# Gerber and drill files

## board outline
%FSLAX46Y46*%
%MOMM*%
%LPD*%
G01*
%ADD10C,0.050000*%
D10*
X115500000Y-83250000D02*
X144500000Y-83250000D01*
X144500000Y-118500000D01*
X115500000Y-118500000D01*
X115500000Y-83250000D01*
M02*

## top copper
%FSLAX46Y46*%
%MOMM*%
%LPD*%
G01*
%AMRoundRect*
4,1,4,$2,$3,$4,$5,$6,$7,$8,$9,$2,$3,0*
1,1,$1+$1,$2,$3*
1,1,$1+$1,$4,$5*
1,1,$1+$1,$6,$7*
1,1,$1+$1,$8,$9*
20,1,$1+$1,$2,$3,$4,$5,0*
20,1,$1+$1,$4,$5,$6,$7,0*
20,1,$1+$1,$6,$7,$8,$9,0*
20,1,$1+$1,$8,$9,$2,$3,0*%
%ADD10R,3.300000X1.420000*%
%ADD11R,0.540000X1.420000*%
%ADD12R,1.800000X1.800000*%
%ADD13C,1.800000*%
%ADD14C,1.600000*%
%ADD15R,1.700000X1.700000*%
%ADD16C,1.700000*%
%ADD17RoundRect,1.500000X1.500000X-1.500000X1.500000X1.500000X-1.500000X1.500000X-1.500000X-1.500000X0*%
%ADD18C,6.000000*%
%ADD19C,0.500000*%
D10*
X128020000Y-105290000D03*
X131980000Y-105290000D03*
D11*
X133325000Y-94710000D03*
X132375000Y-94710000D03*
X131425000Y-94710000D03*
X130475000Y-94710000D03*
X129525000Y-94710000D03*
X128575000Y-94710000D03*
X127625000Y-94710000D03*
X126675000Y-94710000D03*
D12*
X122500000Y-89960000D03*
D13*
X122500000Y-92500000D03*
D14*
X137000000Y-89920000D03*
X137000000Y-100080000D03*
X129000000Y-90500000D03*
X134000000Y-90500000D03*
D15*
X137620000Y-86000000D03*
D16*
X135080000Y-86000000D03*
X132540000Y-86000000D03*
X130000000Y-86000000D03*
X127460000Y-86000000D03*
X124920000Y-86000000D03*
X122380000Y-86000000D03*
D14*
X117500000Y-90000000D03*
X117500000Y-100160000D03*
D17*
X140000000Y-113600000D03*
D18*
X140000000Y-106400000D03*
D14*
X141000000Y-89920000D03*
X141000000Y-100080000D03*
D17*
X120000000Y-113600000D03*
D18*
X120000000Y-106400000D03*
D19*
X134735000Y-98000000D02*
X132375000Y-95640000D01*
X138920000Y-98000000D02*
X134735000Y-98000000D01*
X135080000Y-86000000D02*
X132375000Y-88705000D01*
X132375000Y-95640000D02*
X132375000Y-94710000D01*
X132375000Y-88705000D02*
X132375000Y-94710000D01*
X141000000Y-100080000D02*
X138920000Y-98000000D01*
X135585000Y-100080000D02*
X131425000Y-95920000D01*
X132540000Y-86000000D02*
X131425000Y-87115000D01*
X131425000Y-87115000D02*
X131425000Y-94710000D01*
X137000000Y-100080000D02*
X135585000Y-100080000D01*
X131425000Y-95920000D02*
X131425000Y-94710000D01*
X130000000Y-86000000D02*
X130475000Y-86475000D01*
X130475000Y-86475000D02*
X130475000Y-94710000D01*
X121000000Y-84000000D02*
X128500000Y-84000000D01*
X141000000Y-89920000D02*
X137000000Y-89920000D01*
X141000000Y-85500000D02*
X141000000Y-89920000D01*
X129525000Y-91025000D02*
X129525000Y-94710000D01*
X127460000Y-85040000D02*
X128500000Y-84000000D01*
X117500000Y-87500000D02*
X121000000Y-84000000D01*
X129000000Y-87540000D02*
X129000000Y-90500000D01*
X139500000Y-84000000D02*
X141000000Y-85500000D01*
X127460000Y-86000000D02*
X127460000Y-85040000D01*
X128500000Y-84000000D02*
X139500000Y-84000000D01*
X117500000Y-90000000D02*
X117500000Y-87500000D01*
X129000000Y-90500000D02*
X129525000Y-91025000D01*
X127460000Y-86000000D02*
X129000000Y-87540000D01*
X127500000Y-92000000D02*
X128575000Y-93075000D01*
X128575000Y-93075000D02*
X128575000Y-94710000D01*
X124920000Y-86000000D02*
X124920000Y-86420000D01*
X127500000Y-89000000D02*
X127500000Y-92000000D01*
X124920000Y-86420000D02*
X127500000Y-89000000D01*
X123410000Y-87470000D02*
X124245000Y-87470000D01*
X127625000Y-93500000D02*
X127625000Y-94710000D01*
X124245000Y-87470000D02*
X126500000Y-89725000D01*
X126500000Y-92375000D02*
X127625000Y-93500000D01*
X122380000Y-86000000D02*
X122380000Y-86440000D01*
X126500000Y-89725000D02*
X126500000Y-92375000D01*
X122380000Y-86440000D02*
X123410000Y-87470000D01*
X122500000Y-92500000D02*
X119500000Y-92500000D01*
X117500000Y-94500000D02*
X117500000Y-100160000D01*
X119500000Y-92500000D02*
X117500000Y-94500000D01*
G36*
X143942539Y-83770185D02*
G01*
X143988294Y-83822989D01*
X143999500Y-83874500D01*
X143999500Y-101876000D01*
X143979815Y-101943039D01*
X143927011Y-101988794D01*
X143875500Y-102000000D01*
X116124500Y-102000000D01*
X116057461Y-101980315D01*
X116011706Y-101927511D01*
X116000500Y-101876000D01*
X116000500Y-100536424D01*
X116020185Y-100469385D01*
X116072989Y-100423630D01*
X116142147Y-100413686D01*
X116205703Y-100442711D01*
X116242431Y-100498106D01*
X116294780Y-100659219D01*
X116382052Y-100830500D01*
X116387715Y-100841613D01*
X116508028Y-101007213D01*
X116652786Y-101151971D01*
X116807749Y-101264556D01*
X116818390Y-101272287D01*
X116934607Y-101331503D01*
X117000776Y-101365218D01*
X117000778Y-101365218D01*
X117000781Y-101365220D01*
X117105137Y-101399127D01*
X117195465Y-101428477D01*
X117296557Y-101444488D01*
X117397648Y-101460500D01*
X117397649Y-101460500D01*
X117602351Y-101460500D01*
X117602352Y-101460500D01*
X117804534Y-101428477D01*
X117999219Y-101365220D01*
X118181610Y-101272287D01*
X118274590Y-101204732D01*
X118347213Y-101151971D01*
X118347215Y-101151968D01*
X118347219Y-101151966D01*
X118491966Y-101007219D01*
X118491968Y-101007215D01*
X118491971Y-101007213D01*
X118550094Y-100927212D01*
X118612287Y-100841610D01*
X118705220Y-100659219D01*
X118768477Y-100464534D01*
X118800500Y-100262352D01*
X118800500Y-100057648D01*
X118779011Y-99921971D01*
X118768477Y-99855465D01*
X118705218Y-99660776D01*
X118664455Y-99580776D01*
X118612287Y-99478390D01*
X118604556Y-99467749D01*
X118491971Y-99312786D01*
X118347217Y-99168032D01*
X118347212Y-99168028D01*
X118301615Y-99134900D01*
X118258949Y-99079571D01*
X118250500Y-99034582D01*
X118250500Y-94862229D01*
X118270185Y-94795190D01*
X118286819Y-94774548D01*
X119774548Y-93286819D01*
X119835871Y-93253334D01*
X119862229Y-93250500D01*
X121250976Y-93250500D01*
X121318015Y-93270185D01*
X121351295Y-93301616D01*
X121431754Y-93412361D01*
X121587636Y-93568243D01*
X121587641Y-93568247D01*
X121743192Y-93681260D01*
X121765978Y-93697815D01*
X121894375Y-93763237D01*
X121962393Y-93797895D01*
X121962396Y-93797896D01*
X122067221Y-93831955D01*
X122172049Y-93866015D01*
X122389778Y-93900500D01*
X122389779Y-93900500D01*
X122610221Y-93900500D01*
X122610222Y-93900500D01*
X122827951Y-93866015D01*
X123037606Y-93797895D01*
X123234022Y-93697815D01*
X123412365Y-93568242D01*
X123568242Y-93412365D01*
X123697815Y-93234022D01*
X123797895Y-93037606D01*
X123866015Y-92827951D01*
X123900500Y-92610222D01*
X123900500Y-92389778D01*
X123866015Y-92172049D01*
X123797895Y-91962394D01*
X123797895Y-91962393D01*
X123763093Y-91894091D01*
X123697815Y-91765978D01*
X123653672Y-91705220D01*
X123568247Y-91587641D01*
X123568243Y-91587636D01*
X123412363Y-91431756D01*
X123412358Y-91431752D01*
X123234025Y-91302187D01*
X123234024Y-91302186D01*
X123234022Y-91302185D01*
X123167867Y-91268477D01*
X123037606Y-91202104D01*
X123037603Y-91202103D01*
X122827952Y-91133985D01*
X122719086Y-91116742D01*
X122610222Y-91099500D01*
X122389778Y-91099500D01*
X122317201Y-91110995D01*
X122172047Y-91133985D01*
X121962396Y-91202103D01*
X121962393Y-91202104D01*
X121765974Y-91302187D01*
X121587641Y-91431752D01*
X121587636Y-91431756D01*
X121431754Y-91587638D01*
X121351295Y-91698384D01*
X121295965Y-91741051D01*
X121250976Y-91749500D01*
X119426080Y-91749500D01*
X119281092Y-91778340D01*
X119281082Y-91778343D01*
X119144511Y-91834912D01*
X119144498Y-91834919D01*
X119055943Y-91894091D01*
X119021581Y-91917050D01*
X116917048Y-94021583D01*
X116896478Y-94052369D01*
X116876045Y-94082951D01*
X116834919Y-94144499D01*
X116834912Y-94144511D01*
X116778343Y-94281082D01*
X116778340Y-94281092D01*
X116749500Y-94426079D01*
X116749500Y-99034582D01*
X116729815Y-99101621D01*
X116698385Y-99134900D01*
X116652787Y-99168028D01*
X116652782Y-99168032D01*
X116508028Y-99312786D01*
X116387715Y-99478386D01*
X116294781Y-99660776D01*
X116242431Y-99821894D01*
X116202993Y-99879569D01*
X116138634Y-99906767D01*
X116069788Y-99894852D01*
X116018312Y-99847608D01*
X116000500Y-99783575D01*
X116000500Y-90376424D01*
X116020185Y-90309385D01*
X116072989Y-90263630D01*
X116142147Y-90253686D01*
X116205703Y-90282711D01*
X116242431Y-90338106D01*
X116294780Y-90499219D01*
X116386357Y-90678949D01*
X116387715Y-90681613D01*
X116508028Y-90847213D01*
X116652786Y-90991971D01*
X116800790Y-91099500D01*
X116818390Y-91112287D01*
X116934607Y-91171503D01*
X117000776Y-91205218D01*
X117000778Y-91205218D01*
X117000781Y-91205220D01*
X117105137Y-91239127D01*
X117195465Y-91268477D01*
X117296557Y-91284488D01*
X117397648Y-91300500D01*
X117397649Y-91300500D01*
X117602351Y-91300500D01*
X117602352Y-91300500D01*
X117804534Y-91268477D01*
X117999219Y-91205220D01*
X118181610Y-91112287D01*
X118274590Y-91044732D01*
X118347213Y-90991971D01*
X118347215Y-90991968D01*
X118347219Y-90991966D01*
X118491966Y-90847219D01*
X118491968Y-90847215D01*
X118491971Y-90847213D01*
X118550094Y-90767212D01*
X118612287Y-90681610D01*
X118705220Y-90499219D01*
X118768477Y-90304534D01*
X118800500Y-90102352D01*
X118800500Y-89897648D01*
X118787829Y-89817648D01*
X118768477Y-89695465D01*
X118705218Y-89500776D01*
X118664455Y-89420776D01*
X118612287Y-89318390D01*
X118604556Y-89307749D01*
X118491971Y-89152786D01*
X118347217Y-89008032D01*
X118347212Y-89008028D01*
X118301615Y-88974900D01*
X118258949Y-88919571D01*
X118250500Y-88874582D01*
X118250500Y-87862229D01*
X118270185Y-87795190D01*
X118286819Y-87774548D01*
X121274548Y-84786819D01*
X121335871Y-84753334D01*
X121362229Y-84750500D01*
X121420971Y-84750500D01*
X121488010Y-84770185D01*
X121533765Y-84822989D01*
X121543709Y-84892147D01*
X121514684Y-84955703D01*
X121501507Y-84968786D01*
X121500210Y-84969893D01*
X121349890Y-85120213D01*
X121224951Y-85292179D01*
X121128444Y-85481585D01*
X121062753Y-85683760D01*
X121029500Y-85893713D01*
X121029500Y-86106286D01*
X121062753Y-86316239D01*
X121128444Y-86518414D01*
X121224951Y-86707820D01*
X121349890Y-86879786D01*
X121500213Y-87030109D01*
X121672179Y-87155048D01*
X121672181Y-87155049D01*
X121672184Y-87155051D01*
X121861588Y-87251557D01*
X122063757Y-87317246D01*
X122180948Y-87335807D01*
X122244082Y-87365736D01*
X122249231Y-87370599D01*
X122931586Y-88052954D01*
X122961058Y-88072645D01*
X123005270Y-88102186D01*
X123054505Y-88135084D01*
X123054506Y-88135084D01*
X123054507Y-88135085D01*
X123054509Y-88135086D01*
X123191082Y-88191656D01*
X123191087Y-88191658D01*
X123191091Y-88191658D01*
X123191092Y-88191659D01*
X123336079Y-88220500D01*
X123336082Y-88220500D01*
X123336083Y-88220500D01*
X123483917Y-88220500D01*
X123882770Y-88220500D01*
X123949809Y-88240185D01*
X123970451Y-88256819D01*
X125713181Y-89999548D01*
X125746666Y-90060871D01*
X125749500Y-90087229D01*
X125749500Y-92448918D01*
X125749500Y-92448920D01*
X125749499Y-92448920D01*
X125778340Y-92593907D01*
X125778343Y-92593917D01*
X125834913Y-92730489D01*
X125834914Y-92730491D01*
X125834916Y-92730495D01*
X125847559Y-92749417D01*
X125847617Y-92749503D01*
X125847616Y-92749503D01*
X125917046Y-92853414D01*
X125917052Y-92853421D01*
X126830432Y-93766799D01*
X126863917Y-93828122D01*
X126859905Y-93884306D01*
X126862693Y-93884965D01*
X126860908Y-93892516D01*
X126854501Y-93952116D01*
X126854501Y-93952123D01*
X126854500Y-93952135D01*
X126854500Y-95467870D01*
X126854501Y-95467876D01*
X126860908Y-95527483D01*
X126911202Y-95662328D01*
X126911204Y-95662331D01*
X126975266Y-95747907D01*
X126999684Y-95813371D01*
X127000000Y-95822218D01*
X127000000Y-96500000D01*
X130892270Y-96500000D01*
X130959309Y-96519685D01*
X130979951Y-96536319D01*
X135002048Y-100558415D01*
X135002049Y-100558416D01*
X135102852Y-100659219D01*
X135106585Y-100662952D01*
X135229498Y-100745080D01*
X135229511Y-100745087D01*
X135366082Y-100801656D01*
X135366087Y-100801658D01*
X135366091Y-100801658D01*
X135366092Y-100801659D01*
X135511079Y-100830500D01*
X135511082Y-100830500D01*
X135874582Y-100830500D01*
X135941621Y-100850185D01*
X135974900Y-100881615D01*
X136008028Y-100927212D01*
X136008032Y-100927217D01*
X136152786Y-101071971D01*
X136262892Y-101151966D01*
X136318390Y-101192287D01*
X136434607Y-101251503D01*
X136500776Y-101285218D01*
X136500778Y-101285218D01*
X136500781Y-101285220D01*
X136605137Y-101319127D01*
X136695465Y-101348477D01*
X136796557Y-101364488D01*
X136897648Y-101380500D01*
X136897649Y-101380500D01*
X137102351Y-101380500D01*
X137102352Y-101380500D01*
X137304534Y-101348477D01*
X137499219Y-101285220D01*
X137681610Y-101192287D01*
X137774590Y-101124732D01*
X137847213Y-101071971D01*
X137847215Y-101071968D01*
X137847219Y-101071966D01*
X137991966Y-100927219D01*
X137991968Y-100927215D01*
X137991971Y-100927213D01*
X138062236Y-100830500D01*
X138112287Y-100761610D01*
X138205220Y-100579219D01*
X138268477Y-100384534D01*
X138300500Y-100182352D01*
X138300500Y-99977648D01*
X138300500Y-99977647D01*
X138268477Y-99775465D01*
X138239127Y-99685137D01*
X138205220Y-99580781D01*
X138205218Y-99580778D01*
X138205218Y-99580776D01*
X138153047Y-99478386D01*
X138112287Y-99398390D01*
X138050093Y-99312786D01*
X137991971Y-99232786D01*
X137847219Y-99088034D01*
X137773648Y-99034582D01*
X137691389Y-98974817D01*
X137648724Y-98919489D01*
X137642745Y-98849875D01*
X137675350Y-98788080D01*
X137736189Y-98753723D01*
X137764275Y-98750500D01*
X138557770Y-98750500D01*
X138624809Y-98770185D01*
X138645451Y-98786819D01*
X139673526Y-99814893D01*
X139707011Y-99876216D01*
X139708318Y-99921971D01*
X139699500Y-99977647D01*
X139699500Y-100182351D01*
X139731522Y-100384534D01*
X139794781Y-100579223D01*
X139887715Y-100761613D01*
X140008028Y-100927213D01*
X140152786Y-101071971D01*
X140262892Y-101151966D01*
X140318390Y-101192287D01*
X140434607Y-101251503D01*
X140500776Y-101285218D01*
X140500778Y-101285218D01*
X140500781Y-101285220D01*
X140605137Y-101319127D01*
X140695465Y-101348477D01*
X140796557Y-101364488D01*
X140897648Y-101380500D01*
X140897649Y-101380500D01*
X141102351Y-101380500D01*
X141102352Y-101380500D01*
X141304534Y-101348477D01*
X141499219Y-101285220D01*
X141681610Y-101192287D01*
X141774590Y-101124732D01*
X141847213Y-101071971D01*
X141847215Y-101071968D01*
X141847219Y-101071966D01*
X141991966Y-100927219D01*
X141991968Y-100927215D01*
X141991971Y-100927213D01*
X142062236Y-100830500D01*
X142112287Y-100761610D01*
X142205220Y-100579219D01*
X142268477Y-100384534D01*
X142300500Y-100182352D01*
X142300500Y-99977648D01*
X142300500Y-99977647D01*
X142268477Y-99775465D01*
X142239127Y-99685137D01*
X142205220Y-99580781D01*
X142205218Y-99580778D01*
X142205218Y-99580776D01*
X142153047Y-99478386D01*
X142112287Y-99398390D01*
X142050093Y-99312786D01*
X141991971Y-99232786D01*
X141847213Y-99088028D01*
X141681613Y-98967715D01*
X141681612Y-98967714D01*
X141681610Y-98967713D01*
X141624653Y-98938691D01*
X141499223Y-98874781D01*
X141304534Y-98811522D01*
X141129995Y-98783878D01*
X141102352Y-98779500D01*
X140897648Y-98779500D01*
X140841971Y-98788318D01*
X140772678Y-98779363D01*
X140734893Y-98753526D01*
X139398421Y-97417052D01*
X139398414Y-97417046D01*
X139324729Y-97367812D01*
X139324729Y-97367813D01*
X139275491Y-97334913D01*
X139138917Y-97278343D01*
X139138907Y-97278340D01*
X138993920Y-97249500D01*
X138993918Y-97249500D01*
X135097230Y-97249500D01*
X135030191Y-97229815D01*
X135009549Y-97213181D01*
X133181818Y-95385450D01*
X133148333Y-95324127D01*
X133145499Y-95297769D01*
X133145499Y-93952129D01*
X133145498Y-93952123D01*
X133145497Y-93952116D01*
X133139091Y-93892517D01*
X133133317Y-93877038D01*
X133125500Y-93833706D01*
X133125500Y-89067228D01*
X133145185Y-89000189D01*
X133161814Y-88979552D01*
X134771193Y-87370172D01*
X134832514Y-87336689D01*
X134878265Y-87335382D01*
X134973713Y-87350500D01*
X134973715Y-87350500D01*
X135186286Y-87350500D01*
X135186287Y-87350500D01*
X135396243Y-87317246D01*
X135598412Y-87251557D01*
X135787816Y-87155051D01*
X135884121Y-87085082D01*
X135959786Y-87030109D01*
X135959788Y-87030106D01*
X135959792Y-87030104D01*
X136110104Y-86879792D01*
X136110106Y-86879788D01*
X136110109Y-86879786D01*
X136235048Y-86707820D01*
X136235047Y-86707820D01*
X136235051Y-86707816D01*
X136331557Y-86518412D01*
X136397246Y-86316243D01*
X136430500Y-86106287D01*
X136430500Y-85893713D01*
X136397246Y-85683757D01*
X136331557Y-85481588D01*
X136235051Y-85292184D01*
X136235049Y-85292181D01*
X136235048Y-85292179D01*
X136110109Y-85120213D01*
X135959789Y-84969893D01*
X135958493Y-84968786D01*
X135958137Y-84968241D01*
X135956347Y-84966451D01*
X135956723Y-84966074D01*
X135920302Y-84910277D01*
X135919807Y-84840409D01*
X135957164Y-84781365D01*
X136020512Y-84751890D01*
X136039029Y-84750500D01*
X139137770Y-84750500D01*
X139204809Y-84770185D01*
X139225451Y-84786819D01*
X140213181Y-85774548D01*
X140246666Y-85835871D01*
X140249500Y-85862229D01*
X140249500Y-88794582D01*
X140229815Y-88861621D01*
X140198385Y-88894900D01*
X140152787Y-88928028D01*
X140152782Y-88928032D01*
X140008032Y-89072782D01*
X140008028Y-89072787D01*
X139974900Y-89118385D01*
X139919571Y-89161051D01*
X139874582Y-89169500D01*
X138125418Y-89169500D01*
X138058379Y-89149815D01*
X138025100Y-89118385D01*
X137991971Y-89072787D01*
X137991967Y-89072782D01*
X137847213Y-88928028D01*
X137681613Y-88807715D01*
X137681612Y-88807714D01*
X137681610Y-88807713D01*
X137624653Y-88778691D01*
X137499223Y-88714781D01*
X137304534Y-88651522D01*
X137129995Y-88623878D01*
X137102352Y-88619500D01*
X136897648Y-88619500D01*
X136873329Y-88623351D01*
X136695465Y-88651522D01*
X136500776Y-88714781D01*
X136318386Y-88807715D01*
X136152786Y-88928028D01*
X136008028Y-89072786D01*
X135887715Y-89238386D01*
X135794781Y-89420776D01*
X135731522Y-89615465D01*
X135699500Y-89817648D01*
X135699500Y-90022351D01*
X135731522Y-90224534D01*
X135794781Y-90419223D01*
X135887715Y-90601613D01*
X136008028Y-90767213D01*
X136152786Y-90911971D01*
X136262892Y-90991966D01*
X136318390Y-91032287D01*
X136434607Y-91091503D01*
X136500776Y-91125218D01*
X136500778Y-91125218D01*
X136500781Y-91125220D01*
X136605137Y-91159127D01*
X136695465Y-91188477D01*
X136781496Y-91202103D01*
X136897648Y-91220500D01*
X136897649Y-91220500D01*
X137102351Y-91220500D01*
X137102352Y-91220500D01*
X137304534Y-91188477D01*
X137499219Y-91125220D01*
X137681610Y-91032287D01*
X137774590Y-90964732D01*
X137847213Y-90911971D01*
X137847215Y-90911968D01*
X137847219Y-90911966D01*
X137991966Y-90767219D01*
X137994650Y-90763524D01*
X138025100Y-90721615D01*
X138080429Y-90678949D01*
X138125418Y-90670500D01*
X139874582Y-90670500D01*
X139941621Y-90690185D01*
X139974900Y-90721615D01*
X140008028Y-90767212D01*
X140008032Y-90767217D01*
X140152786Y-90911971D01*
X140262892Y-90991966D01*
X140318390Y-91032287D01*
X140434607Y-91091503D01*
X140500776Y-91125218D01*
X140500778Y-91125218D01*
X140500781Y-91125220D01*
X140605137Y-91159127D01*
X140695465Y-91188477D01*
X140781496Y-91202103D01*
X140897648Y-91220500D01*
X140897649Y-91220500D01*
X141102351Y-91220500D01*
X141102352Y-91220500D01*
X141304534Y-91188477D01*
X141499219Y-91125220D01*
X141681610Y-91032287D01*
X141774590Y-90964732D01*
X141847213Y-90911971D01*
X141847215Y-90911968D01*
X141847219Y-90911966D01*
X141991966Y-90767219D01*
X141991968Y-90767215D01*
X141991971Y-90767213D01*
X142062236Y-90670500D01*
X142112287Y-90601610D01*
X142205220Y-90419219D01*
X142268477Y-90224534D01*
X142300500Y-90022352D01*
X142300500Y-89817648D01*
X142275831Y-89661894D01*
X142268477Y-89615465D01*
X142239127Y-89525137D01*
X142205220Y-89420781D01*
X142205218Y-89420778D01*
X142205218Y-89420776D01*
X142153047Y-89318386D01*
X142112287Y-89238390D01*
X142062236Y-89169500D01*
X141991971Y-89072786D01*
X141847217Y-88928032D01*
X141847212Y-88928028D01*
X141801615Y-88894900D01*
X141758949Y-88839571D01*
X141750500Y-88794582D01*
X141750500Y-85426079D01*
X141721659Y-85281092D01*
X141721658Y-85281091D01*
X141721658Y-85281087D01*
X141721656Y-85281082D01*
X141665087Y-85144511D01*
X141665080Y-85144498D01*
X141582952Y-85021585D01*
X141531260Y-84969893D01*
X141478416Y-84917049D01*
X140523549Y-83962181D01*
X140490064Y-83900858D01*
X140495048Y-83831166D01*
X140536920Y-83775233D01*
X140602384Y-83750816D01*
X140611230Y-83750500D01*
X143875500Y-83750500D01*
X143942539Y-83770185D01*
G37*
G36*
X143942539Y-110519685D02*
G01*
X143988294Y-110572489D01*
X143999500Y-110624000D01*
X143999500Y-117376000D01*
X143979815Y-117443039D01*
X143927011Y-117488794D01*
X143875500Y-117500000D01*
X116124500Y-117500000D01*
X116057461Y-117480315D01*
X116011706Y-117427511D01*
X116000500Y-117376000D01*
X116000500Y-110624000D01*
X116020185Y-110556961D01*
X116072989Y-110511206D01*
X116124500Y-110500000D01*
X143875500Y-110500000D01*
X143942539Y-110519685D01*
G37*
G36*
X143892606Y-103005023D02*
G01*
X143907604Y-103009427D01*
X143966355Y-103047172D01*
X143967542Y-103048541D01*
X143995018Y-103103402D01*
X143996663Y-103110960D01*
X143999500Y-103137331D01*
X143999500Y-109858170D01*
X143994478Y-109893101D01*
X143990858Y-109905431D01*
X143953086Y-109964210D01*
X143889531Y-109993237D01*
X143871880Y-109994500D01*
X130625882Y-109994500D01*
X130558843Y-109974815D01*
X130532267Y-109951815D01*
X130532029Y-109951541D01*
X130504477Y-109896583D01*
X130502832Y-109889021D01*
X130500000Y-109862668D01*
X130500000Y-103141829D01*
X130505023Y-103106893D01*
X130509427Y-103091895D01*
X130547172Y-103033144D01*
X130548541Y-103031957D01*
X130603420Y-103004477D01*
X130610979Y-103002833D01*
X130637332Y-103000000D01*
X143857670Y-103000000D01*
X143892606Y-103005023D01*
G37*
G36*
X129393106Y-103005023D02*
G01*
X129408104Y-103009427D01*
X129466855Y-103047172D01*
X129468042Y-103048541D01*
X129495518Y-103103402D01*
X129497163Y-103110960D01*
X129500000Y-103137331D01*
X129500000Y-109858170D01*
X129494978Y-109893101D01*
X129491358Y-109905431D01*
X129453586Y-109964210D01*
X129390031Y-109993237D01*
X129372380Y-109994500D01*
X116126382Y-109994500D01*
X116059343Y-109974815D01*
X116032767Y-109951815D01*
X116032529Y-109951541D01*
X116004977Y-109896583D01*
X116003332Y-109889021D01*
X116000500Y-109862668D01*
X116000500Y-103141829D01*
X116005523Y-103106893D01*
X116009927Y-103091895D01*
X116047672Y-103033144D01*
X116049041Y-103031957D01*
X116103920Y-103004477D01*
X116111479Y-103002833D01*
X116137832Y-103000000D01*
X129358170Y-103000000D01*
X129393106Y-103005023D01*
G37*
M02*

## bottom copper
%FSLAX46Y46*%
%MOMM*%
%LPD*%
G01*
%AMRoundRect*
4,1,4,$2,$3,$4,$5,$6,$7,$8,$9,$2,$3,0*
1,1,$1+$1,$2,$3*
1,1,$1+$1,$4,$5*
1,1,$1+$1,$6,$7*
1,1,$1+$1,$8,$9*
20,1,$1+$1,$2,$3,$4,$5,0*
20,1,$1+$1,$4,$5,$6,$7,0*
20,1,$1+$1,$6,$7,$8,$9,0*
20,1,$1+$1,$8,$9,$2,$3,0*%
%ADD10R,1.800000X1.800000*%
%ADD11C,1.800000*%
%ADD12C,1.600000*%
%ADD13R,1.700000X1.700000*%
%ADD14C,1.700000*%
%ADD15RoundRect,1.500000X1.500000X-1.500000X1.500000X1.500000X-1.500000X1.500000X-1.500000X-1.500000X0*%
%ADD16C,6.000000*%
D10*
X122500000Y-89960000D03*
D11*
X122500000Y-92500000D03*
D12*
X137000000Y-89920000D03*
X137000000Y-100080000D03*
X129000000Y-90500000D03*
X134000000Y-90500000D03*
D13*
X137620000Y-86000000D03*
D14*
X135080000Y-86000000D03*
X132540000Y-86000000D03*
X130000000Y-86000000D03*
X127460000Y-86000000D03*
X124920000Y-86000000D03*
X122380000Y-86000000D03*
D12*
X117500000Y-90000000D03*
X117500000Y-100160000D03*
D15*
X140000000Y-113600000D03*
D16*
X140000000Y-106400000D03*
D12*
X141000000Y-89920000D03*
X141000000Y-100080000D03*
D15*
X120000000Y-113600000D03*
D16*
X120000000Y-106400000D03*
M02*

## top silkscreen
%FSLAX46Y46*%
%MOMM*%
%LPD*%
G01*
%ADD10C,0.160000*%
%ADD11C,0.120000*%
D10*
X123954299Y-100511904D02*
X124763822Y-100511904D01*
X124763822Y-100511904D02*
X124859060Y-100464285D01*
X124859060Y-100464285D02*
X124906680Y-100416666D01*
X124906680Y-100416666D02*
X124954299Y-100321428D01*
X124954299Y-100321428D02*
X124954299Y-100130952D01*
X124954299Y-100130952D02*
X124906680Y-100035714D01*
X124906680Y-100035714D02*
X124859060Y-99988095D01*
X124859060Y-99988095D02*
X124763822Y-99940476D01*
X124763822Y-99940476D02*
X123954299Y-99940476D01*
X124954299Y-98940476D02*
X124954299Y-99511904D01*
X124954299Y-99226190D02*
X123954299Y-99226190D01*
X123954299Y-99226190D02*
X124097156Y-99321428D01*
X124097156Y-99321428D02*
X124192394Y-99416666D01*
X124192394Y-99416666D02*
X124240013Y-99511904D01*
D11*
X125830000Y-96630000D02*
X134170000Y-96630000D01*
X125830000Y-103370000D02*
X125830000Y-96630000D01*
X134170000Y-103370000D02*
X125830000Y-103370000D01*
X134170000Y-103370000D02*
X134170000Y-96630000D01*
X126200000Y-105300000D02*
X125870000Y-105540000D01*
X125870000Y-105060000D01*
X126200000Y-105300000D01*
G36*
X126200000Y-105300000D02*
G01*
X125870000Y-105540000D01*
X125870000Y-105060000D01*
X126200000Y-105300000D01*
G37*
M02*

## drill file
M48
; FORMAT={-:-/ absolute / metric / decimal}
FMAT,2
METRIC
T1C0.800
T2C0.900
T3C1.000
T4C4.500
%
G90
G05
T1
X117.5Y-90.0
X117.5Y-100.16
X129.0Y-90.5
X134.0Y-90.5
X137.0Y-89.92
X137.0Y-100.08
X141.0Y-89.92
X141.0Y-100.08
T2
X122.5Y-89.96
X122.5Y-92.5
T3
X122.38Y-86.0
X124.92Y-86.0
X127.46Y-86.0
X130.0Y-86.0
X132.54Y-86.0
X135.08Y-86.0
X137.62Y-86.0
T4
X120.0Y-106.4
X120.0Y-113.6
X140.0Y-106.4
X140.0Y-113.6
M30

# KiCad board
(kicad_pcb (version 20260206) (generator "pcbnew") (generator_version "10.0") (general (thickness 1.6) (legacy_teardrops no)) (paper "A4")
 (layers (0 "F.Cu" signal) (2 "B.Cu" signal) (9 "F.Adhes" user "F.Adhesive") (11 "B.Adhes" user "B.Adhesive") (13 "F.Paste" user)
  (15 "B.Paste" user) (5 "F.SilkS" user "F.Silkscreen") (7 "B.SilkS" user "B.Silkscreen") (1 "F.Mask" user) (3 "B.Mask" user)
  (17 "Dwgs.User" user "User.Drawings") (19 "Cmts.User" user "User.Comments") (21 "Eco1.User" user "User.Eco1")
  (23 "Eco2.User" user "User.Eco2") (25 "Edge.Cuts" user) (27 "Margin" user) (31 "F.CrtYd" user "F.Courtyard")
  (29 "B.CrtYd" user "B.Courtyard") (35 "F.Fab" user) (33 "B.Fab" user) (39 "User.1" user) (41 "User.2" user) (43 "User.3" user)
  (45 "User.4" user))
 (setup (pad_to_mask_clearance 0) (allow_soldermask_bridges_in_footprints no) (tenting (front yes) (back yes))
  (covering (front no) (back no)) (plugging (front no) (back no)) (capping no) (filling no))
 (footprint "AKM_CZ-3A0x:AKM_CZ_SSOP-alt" (layer "F.Cu") (at 130 100 90)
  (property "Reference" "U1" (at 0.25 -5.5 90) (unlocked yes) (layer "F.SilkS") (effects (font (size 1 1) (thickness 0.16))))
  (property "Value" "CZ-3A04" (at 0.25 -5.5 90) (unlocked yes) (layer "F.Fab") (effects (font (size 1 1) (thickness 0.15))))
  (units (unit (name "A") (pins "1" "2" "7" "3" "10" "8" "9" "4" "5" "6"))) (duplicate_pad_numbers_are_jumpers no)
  (fp_line (start 3.37 -4.17) (end 3.37 4.17) (stroke (width 0.12) (type solid)) (layer "F.SilkS"))
  (fp_line (start -3.37 -4.17) (end 3.37 -4.17) (stroke (width 0.12) (type solid)) (layer "F.SilkS"))
  (fp_line (start -3.37 4.17) (end -3.37 -4.17) (stroke (width 0.12) (type solid)) (layer "F.SilkS"))
  (fp_line (start -3.37 4.17) (end 3.37 4.17) (stroke (width 0.12) (type solid)) (layer "F.SilkS"))
  (fp_poly
   (pts (xy -5.3 -3.8) (xy -5.54 -4.13) (xy -5.06 -4.13) (xy -5.3 -3.8)) (stroke (width 0.12) (type solid)) (fill yes) (layer "F.SilkS"))
  (pad "1" smd rect (at -5.29 -1.98 270) (size 1.42 3.3) (layers "F.Cu" "F.Mask" "F.Paste") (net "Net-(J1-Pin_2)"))
  (pad "2" smd rect (at -5.29 1.98 270) (size 1.42 3.3) (layers "F.Cu" "F.Mask" "F.Paste") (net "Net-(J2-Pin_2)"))
  (pad "3" smd rect (at 5.29 3.325 270) (size 1.42 0.54) (layers "F.Cu" "F.Mask" "F.Paste") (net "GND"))
  (pad "4" smd rect (at 5.29 2.375 270) (size 1.42 0.54) (layers "F.Cu" "F.Mask" "F.Paste") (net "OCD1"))
  (pad "5" smd rect (at 5.29 1.425 270) (size 1.42 0.54) (layers "F.Cu" "F.Mask" "F.Paste") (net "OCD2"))
  (pad "6" smd rect (at 5.29 0.475 270) (size 1.42 0.54) (layers "F.Cu" "F.Mask" "F.Paste") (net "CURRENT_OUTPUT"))
  (pad "7" smd rect (at 5.29 -0.475 270) (size 1.42 0.54) (layers "F.Cu" "F.Mask" "F.Paste") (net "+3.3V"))
  (pad "8" smd rect (at 5.29 -1.425 270) (size 1.42 0.54) (layers "F.Cu" "F.Mask" "F.Paste") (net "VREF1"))
  (pad "9" smd rect (at 5.29 -2.375 270) (size 1.42 0.54) (layers "F.Cu" "F.Mask" "F.Paste") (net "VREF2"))
  (pad "10" smd rect (at 5.29 -3.325 270) (size 1.42 0.54) (layers "F.Cu" "F.Mask" "F.Paste") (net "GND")))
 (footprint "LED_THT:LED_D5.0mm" (layer "B.Cu") (at 122.5 89.96 -90)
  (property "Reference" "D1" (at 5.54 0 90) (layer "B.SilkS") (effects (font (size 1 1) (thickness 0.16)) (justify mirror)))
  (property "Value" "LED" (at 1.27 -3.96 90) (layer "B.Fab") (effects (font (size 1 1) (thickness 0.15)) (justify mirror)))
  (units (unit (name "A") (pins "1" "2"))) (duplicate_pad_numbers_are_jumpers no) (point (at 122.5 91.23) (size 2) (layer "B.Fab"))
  (pad "1" thru_hole rect (at 0 0 270) (size 1.8 1.8) (drill 0.9) (layers "*.Cu" "*.Mask") (remove_unused_layers no) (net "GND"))
  (pad "2" thru_hole circle (at 2.54 0 270) (size 1.8 1.8) (drill 0.9) (layers "*.Cu" "*.Mask") (remove_unused_layers no) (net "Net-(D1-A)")))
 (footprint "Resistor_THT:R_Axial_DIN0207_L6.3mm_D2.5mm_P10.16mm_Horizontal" (layer "B.Cu") (at 137 89.92 -90)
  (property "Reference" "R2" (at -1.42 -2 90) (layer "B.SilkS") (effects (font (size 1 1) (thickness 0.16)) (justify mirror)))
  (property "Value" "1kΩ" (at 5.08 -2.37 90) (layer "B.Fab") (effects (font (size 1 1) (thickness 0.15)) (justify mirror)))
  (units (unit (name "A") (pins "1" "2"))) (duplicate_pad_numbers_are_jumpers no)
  (pad "1" thru_hole circle (at 0 0 270) (size 1.6 1.6) (drill 0.8) (layers "*.Cu" "*.Mask") (remove_unused_layers no) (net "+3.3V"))
  (pad "2" thru_hole circle (at 10.16 0 270) (size 1.6 1.6) (drill 0.8) (layers "*.Cu" "*.Mask") (remove_unused_layers no) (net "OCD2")))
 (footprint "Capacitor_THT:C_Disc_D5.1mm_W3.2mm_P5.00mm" (layer "B.Cu") (at 129 90.5)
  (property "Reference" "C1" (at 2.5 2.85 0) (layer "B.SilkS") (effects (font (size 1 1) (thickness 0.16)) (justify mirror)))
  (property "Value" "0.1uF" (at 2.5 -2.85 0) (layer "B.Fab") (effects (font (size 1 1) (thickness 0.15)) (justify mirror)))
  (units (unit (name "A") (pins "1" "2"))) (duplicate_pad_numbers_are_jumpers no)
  (pad "1" thru_hole circle (at 0 0) (size 1.6 1.6) (drill 0.8) (layers "*.Cu" "*.Mask") (remove_unused_layers no) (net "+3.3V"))
  (pad "2" thru_hole circle (at 5 0) (size 1.6 1.6) (drill 0.8) (layers "*.Cu" "*.Mask") (remove_unused_layers no) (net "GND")))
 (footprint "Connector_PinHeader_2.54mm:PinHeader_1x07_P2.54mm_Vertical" (layer "B.Cu") (at 137.62 86 90)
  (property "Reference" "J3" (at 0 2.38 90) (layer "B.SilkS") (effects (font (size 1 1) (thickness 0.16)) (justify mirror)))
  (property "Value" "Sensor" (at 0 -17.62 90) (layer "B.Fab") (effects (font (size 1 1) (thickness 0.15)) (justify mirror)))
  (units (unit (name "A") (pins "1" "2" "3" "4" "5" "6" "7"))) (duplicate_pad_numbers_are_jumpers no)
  (pad "1" thru_hole rect (at 0 0 90) (size 1.7 1.7) (drill 1) (layers "*.Cu" "*.Mask") (remove_unused_layers no) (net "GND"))
  (pad "2" thru_hole circle (at 0 -2.54 90) (size 1.7 1.7) (drill 1) (layers "*.Cu" "*.Mask") (remove_unused_layers no) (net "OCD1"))
  (pad "3" thru_hole circle (at 0 -5.08 90) (size 1.7 1.7) (drill 1) (layers "*.Cu" "*.Mask") (remove_unused_layers no) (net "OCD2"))
  (pad "4" thru_hole circle (at 0 -7.62 90) (size 1.7 1.7) (drill 1) (layers "*.Cu" "*.Mask") (remove_unused_layers no)
   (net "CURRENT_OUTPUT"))
  (pad "5" thru_hole circle (at 0 -10.16 90) (size 1.7 1.7) (drill 1) (layers "*.Cu" "*.Mask") (remove_unused_layers no) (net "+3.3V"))
  (pad "6" thru_hole circle (at 0 -12.7 90) (size 1.7 1.7) (drill 1) (layers "*.Cu" "*.Mask") (remove_unused_layers no) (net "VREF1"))
  (pad "7" thru_hole circle (at 0 -15.24 90) (size 1.7 1.7) (drill 1) (layers "*.Cu" "*.Mask") (remove_unused_layers no) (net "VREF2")))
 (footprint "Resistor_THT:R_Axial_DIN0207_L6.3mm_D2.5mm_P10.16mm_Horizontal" (layer "B.Cu") (at 117.5 90 -90)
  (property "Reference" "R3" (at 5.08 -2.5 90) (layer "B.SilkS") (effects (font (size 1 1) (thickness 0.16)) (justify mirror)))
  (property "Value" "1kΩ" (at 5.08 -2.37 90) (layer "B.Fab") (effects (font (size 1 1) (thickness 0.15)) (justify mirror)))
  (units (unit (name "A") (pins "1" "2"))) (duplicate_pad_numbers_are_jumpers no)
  (pad "1" thru_hole circle (at 0 0 270) (size 1.6 1.6) (drill 0.8) (layers "*.Cu" "*.Mask") (remove_unused_layers no) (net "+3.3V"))
  (pad "2" thru_hole circle (at 10.16 0 270) (size 1.6 1.6) (drill 0.8) (layers "*.Cu" "*.Mask") (remove_unused_layers no)
   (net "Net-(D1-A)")))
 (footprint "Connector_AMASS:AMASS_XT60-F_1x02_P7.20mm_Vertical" (layer "B.Cu") (at 140 113.6 90)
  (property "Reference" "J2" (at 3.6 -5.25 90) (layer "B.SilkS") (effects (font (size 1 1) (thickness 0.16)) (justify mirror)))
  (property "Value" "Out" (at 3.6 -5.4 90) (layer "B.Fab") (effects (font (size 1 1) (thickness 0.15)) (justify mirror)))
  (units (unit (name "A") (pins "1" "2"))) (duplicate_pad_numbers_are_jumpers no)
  (pad "1" thru_hole roundrect (at 0 0 90) (size 6 6) (drill 4.5) (layers "*.Cu" "*.Mask") (remove_unused_layers no) (roundrect_rratio 0.25)
   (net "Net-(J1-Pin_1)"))
  (pad "2" thru_hole circle (at 7.2 0 90) (size 6 6) (drill 4.5) (layers "*.Cu" "*.Mask") (remove_unused_layers no) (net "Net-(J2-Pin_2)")))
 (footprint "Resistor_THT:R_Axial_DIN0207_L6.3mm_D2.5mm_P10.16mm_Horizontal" (layer "B.Cu") (at 141 89.92 -90)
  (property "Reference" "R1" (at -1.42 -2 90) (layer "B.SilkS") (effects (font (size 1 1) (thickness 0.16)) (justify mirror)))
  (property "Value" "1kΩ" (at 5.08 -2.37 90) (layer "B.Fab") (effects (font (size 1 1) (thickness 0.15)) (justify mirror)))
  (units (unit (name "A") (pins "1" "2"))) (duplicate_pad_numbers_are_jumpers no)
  (pad "1" thru_hole circle (at 0 0 270) (size 1.6 1.6) (drill 0.8) (layers "*.Cu" "*.Mask") (remove_unused_layers no) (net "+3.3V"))
  (pad "2" thru_hole circle (at 10.16 0 270) (size 1.6 1.6) (drill 0.8) (layers "*.Cu" "*.Mask") (remove_unused_layers no) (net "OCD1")))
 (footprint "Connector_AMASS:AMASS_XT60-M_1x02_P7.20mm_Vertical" (layer "B.Cu") (at 120 113.6 90)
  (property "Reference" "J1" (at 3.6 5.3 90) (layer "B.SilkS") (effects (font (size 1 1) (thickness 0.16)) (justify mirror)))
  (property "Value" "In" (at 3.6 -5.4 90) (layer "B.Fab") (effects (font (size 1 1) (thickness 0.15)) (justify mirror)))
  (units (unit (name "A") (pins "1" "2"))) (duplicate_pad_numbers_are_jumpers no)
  (pad "1" thru_hole roundrect (at 0 0 90) (size 6 6) (drill 4.5) (layers "*.Cu" "*.Mask") (remove_unused_layers no) (roundrect_rratio 0.25)
   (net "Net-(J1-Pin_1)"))
  (pad "2" thru_hole circle (at 7.2 0 90) (size 6 6) (drill 4.5) (layers "*.Cu" "*.Mask") (remove_unused_layers no) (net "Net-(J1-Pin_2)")))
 (gr_rect (start 115.5 83.25) (end 144.5 118.5) (stroke (width 0.05) (type default)) (fill no) (layer "Edge.Cuts"))
 (segment (start 134.735 98) (end 132.375 95.64) (width 0.5) (layer "F.Cu") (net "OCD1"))
 (segment (start 138.92 98) (end 134.735 98) (width 0.5) (layer "F.Cu") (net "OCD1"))
 (segment (start 135.08 86) (end 132.375 88.705) (width 0.5) (layer "F.Cu") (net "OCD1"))
 (segment (start 132.375 95.64) (end 132.375 94.71) (width 0.5) (layer "F.Cu") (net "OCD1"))
 (segment (start 132.375 88.705) (end 132.375 94.71) (width 0.5) (layer "F.Cu") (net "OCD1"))
 (segment (start 141 100.08) (end 138.92 98) (width 0.5) (layer "F.Cu") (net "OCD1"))
 (segment (start 135.585 100.08) (end 131.425 95.92) (width 0.5) (layer "F.Cu") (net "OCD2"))
 (segment (start 132.54 86) (end 131.425 87.115) (width 0.5) (layer "F.Cu") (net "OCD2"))
 (segment (start 131.425 87.115) (end 131.425 94.71) (width 0.5) (layer "F.Cu") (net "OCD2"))
 (segment (start 137 100.08) (end 135.585 100.08) (width 0.5) (layer "F.Cu") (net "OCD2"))
 (segment (start 131.425 95.92) (end 131.425 94.71) (width 0.5) (layer "F.Cu") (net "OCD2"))
 (segment (start 130 86) (end 130.475 86.475) (width 0.5) (layer "F.Cu") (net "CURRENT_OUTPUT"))
 (segment (start 130.475 86.475) (end 130.475 94.71) (width 0.5) (layer "F.Cu") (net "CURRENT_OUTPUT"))
 (segment (start 121 84) (end 128.5 84) (width 0.5) (layer "F.Cu") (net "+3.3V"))
 (segment (start 141 89.92) (end 137 89.92) (width 0.5) (layer "F.Cu") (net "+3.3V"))
 (segment (start 141 85.5) (end 141 89.92) (width 0.5) (layer "F.Cu") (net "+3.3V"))
 (segment (start 129.525 91.025) (end 129.525 94.71) (width 0.5) (layer "F.Cu") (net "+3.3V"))
 (segment (start 127.46 85.04) (end 128.5 84) (width 0.5) (layer "F.Cu") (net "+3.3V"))
 (segment (start 117.5 87.5) (end 121 84) (width 0.5) (layer "F.Cu") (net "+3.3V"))
 (segment (start 129 87.54) (end 129 90.5) (width 0.5) (layer "F.Cu") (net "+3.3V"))
 (segment (start 139.5 84) (end 141 85.5) (width 0.5) (layer "F.Cu") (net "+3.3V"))
 (segment (start 127.46 86) (end 127.46 85.04) (width 0.5) (layer "F.Cu") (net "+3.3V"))
 (segment (start 128.5 84) (end 139.5 84) (width 0.5) (layer "F.Cu") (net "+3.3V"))
 (segment (start 117.5 90) (end 117.5 87.5) (width 0.5) (layer "F.Cu") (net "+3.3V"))
 (segment (start 129 90.5) (end 129.525 91.025) (width 0.5) (layer "F.Cu") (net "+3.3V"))
 (segment (start 127.46 86) (end 129 87.54) (width 0.5) (layer "F.Cu") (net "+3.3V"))
 (segment (start 127.5 92) (end 128.575 93.075) (width 0.5) (layer "F.Cu") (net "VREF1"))
 (segment (start 128.575 93.075) (end 128.575 94.71) (width 0.5) (layer "F.Cu") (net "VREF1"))
 (segment (start 124.92 86) (end 124.92 86.42) (width 0.5) (layer "F.Cu") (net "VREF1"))
 (segment (start 127.5 89) (end 127.5 92) (width 0.5) (layer "F.Cu") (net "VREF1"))
 (segment (start 124.92 86.42) (end 127.5 89) (width 0.5) (layer "F.Cu") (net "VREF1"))
 (segment (start 123.41 87.47) (end 124.245 87.47) (width 0.5) (layer "F.Cu") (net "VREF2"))
 (segment (start 127.625 93.5) (end 127.625 94.71) (width 0.5) (layer "F.Cu") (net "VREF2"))
 (segment (start 124.245 87.47) (end 126.5 89.725) (width 0.5) (layer "F.Cu") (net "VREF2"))
 (segment (start 126.5 92.375) (end 127.625 93.5) (width 0.5) (layer "F.Cu") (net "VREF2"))
 (segment (start 122.38 86) (end 122.38 86.44) (width 0.5) (layer "F.Cu") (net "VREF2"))
 (segment (start 126.5 89.725) (end 126.5 92.375) (width 0.5) (layer "F.Cu") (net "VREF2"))
 (segment (start 122.38 86.44) (end 123.41 87.47) (width 0.5) (layer "F.Cu") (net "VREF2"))
 (segment (start 122.5 92.5) (end 119.5 92.5) (width 0.5) (layer "F.Cu") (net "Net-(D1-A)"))
 (segment (start 117.5 94.5) (end 117.5 100.16) (width 0.5) (layer "F.Cu") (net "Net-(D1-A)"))
 (segment (start 119.5 92.5) (end 117.5 94.5) (width 0.5) (layer "F.Cu") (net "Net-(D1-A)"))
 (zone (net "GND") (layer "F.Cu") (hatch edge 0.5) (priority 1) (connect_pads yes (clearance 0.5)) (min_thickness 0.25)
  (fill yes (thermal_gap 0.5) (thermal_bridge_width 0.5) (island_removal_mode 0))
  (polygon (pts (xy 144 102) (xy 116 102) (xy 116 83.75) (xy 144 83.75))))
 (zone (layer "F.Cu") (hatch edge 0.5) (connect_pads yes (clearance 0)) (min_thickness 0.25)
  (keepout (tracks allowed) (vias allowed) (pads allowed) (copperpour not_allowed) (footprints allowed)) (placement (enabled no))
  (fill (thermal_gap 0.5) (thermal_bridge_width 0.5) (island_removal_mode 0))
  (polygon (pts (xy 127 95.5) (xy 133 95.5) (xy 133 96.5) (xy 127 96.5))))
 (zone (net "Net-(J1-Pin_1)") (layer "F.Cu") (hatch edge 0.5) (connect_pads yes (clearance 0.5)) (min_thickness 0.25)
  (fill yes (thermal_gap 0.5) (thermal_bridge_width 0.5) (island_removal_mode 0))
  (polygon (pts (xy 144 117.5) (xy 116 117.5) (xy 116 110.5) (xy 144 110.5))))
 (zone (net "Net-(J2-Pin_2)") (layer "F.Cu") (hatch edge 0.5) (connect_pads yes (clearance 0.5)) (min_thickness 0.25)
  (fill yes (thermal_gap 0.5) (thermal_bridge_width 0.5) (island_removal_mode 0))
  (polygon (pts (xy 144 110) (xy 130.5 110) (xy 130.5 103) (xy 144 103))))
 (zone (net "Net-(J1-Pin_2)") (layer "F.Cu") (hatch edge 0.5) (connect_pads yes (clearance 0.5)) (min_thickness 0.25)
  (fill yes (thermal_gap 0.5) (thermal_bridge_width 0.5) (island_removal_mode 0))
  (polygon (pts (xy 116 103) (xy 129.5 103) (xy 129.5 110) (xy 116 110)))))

